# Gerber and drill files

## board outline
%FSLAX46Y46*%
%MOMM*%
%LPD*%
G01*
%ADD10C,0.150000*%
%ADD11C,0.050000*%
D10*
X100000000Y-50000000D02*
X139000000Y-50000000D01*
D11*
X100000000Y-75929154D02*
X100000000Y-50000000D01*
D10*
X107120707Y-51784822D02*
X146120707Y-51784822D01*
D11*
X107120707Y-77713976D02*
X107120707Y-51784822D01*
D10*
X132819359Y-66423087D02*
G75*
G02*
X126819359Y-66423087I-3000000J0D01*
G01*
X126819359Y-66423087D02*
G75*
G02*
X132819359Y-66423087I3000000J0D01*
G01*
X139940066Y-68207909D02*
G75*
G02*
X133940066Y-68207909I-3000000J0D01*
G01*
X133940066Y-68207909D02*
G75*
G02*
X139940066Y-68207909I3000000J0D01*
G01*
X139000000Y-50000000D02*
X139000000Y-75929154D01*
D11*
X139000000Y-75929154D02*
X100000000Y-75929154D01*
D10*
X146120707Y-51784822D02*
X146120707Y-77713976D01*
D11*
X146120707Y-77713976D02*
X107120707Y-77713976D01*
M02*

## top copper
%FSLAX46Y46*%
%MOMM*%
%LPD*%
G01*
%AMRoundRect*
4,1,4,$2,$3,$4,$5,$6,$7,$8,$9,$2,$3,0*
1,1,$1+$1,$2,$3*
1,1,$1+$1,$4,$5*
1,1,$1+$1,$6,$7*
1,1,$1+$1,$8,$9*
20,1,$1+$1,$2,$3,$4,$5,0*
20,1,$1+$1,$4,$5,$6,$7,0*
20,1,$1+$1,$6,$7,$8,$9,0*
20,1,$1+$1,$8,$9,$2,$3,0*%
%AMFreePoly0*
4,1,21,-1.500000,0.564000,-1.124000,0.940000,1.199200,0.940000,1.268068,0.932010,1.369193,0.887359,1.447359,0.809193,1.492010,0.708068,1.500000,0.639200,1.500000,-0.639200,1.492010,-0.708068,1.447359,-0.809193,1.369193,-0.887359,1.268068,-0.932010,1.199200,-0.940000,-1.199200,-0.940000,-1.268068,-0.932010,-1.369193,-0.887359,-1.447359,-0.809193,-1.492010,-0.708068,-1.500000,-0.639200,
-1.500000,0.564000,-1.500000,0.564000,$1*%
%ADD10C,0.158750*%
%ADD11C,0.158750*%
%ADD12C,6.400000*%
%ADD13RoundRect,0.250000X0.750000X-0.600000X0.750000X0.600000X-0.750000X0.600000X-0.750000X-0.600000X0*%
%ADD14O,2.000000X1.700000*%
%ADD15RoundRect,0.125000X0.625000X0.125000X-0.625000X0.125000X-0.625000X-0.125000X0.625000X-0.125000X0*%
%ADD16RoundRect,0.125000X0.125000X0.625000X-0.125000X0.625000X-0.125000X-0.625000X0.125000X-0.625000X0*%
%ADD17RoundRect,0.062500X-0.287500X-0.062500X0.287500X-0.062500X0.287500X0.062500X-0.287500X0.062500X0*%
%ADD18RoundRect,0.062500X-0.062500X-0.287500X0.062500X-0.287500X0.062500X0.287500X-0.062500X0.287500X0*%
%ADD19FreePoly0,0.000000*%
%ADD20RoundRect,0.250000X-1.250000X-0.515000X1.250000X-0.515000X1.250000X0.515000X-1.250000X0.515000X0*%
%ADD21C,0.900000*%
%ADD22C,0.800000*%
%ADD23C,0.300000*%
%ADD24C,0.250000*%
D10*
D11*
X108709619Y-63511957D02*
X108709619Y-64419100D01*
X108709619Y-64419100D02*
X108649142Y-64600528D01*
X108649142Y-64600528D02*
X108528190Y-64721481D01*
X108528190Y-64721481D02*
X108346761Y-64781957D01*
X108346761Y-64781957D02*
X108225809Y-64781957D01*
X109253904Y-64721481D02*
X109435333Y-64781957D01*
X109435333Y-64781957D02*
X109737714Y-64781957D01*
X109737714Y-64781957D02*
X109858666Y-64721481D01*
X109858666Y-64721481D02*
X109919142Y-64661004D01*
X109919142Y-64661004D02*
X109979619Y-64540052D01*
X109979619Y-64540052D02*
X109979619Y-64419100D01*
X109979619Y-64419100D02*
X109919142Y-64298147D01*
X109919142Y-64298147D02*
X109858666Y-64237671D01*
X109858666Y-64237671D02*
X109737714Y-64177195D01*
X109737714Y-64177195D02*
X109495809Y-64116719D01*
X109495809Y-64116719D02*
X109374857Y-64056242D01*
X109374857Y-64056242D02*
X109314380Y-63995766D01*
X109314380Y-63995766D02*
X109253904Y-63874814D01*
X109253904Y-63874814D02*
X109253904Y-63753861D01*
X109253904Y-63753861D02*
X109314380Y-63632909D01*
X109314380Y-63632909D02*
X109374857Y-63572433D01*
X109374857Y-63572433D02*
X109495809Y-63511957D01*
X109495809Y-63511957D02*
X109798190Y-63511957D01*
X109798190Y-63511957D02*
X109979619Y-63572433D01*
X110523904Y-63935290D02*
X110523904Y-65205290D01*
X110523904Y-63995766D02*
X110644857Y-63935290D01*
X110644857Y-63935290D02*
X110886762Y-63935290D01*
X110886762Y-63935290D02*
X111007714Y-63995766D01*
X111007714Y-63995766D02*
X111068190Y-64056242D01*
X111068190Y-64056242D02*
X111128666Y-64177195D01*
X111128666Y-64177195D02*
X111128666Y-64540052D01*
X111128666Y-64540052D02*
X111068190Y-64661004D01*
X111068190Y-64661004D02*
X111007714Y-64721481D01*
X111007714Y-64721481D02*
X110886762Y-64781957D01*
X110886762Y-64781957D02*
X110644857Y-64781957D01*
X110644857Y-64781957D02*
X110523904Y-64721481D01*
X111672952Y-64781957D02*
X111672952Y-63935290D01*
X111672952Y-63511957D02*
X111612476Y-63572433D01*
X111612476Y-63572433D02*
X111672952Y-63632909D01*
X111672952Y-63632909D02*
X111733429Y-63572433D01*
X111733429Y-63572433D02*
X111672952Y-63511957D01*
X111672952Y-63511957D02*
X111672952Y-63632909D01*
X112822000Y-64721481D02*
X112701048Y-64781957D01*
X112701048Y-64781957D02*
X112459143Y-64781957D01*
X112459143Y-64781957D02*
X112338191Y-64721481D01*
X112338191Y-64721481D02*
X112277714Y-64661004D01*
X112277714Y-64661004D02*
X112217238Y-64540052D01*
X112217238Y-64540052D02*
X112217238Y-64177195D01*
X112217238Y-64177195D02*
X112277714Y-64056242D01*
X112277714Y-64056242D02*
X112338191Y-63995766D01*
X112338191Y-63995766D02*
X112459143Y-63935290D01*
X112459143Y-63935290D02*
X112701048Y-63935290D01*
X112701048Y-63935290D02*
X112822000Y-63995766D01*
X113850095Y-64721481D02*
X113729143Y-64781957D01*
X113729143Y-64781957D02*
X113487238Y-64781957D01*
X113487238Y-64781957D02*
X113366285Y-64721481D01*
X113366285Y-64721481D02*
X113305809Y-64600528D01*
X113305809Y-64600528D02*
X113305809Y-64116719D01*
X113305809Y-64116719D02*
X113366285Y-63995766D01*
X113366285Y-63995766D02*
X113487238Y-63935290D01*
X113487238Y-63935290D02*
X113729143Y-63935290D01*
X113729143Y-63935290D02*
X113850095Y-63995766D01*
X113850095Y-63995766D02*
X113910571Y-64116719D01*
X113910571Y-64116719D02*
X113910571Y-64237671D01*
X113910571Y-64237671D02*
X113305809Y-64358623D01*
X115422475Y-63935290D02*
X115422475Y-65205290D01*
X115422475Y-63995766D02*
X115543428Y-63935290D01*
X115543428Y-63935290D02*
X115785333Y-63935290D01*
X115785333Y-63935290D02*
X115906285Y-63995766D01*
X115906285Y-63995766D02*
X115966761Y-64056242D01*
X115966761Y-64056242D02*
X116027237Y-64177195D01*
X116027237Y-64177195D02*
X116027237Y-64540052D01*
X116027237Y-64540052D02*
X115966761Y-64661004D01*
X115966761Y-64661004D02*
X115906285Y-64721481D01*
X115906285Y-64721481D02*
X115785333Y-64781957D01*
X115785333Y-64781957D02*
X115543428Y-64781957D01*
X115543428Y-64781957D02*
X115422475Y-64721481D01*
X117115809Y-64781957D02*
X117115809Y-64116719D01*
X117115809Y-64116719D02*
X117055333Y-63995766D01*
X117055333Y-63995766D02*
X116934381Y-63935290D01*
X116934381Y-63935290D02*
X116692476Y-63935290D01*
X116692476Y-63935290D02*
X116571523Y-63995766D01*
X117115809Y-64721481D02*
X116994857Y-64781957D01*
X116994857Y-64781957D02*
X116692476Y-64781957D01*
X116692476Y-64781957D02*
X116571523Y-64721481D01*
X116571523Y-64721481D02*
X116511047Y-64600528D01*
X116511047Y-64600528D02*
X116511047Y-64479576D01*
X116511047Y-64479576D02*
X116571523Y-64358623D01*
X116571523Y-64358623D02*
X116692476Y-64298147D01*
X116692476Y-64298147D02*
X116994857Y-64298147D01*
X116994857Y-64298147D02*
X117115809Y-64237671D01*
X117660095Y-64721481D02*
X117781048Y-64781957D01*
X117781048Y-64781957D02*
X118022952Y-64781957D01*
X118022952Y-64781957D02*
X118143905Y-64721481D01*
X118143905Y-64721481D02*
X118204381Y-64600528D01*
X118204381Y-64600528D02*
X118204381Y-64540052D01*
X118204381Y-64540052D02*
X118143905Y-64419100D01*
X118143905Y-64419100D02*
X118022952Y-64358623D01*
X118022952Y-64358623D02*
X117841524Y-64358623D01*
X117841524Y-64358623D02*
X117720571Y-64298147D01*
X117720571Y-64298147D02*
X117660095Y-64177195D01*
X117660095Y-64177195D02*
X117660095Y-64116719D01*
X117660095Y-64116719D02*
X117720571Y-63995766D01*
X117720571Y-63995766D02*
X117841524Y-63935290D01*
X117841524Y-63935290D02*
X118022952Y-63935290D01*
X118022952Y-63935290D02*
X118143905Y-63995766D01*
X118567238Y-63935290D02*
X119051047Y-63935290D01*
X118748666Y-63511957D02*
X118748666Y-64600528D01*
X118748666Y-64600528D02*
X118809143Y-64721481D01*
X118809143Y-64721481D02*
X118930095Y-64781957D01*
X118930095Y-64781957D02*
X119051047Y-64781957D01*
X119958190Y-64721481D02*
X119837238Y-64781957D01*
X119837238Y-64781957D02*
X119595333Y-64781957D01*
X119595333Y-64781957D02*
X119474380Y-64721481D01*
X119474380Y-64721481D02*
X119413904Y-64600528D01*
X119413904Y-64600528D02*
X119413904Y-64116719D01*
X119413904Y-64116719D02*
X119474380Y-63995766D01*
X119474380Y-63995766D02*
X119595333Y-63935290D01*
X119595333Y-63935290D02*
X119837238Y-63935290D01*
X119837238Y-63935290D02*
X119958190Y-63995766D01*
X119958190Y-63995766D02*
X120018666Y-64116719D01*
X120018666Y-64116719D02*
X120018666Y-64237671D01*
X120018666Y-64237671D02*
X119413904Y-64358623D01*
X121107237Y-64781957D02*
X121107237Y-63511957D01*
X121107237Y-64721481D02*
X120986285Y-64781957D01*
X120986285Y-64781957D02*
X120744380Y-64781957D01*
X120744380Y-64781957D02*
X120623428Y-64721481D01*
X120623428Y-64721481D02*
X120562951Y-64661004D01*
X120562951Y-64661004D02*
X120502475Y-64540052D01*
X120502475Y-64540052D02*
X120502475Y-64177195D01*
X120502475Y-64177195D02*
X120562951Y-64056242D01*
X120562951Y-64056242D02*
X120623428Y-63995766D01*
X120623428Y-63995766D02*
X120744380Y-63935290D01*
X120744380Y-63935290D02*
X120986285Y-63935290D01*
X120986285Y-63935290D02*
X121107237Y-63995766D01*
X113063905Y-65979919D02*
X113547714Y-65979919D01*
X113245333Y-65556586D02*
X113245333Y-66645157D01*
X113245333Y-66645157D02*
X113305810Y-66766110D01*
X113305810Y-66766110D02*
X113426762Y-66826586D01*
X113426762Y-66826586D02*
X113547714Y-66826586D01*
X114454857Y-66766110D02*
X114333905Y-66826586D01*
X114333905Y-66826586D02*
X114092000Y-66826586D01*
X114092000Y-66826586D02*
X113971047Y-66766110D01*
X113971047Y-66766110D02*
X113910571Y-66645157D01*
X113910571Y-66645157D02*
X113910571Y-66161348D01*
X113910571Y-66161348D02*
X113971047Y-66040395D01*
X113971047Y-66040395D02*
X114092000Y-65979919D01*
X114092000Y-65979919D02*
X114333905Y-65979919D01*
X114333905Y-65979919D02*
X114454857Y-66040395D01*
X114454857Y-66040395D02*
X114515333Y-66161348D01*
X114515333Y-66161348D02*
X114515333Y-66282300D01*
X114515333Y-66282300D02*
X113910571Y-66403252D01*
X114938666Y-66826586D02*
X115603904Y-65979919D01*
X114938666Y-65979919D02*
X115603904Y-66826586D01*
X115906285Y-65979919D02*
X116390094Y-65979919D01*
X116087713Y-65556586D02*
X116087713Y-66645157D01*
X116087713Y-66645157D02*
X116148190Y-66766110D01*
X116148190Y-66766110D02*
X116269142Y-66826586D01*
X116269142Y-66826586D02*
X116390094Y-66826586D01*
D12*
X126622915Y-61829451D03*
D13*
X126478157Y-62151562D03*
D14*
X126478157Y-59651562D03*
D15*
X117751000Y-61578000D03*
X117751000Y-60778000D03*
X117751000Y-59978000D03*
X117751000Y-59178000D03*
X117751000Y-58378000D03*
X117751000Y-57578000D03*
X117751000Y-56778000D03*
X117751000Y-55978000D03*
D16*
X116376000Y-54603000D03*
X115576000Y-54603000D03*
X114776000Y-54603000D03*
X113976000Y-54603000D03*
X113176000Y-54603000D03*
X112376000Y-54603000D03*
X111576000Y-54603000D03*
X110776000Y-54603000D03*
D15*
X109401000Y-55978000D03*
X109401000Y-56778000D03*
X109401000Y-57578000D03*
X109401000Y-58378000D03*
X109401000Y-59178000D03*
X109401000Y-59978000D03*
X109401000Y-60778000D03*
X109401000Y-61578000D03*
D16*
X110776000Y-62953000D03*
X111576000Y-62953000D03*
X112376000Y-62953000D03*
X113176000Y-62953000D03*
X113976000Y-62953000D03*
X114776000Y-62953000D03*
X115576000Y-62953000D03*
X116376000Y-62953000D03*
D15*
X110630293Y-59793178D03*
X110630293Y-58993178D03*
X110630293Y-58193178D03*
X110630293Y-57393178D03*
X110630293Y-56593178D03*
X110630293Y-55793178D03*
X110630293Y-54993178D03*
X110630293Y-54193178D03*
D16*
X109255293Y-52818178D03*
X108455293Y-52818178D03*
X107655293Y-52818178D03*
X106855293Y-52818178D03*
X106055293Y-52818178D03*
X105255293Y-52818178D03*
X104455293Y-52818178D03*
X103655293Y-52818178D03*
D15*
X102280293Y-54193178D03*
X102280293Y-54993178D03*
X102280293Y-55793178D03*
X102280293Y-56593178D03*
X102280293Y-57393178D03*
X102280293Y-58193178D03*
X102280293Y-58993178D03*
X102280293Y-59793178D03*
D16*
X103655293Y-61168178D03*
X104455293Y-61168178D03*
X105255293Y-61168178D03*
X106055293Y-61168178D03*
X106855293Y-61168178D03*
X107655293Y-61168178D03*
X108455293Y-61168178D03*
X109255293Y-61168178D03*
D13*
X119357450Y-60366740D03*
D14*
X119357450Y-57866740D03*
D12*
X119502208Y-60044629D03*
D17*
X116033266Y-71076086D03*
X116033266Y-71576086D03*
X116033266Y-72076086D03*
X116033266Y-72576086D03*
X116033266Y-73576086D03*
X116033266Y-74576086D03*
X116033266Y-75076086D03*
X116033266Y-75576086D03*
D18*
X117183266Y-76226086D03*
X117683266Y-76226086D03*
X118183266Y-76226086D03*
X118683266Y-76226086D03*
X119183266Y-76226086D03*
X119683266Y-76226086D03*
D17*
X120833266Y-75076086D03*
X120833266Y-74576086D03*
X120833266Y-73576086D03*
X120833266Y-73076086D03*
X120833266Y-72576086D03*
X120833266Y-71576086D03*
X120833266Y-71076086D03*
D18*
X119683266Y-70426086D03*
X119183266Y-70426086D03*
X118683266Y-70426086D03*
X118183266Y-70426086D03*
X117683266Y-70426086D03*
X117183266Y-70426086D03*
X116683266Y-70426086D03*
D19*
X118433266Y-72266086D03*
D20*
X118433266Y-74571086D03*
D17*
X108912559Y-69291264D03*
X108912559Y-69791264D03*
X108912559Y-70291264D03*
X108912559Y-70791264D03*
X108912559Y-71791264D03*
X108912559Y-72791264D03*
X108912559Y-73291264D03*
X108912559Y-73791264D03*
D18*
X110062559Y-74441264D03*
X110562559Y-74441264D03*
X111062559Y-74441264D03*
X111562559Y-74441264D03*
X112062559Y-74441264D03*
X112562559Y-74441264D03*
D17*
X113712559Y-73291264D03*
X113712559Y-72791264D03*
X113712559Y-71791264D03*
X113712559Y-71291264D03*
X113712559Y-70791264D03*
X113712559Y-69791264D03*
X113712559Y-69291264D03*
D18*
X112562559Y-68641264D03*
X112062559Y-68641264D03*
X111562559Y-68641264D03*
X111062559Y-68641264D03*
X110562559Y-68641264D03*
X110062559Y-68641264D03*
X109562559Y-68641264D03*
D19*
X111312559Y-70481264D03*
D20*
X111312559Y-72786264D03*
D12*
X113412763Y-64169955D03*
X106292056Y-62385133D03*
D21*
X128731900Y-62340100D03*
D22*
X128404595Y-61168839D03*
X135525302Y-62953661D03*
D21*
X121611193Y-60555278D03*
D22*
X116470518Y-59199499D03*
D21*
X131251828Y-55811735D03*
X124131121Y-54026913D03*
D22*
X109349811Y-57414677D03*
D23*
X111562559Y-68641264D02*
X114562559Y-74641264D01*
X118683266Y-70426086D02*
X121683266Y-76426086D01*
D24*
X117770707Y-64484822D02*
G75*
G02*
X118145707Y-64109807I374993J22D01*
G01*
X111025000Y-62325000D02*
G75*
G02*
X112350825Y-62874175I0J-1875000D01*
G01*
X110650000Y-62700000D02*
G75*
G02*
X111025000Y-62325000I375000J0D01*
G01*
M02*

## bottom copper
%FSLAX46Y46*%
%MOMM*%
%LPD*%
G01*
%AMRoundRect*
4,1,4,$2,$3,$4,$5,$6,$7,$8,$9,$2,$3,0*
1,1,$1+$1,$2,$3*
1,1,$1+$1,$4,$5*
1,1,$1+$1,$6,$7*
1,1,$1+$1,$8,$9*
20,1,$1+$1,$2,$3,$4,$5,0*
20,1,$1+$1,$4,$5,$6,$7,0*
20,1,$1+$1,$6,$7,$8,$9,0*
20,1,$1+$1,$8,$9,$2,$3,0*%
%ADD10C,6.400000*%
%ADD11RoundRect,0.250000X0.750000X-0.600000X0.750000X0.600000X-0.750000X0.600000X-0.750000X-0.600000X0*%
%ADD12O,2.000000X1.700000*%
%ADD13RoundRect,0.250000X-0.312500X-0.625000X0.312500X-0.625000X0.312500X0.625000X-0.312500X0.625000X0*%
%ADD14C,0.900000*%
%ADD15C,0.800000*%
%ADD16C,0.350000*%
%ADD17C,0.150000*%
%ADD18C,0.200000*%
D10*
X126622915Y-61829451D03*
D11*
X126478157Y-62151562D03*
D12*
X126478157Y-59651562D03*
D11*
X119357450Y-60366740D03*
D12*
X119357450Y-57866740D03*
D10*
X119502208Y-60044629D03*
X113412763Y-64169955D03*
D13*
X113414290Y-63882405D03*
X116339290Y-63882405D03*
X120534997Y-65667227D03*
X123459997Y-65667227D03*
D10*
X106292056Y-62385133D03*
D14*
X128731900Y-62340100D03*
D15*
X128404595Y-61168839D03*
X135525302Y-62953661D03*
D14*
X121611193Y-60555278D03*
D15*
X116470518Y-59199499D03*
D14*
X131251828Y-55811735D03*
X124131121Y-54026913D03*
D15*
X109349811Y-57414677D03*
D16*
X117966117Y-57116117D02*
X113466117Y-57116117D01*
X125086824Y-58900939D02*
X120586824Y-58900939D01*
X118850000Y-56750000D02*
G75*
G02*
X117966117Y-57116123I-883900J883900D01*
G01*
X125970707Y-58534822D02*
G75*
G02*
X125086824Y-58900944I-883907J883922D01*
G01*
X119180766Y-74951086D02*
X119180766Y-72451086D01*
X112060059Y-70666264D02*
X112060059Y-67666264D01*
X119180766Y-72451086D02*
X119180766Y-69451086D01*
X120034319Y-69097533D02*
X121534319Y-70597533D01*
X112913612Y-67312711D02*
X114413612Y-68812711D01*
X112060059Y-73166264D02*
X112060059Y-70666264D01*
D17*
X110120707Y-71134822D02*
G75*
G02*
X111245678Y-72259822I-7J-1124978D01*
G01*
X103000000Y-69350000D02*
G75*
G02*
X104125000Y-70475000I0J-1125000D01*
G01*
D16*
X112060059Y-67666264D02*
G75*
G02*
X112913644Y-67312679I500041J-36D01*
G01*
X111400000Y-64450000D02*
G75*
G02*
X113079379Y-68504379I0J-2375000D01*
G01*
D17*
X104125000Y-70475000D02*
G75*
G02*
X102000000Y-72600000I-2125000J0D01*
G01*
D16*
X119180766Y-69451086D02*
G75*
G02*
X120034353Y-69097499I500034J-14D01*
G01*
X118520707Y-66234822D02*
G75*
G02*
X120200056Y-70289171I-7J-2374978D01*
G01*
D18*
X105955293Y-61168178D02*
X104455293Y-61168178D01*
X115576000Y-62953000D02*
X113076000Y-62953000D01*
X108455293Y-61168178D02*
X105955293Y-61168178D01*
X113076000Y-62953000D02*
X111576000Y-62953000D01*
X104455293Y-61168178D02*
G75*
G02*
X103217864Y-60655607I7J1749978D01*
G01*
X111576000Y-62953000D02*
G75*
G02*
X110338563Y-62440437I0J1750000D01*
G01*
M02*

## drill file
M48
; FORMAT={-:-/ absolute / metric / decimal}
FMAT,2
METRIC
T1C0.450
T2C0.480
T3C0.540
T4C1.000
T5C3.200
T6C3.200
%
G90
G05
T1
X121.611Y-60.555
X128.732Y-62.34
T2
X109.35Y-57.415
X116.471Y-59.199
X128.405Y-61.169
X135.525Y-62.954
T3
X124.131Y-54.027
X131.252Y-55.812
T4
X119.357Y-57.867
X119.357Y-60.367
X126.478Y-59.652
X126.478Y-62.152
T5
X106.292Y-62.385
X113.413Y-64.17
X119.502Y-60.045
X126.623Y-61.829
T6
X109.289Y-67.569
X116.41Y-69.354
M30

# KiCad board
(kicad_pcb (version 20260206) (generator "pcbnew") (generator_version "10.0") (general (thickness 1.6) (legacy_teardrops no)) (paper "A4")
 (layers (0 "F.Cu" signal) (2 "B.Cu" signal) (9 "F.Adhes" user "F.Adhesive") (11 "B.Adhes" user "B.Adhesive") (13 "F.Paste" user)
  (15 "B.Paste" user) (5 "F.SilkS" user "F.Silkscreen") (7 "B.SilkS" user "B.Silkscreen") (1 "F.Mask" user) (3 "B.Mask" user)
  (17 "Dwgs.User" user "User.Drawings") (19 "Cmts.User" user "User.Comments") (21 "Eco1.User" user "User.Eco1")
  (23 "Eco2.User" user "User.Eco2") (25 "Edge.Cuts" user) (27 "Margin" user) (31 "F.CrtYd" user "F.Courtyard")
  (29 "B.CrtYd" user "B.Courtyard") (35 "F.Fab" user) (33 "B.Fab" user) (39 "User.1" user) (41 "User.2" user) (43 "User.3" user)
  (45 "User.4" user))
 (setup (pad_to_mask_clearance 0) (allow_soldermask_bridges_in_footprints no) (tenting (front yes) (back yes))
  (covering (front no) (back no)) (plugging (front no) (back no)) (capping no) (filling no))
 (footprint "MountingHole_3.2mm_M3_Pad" (layer "F.Cu") (at 126.622915 61.829451)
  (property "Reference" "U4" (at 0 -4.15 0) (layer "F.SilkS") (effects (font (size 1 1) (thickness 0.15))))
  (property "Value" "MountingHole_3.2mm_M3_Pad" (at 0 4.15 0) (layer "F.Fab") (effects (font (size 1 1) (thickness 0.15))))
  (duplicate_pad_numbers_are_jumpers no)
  (pad "1" thru_hole circle (at 0 0) (size 6.4 6.4) (drill 3.2) (layers "*.Cu" "*.Mask") (remove_unused_layers no) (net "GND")
   (zone_connect 2)))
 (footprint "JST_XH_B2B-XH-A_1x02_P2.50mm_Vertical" (layer "F.Cu") (at 126.478157 62.151562 90)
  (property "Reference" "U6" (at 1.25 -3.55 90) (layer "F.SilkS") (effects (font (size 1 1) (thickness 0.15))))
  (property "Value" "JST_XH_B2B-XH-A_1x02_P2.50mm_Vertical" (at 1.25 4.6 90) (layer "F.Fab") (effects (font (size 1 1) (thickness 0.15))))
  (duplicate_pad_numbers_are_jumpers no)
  (pad "1" thru_hole roundrect (at 0 0 90) (size 1.7 2) (drill 1) (layers "*.Cu" "*.Mask") (remove_unused_layers no)
   (roundrect_rratio 0.147059) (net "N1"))
  (pad "2" thru_hole oval (at 2.5 0 90) (size 1.7 2) (drill 1) (layers "*.Cu" "*.Mask") (remove_unused_layers no)))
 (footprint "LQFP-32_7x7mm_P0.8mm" (layer "F.Cu") (at 113.576 58.778 180)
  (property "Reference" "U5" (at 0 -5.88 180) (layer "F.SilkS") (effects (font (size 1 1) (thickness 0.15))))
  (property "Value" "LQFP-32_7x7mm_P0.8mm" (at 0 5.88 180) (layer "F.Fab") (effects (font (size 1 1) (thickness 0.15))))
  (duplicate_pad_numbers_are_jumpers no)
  (pad "1" smd roundrect (at -4.175 -2.8 180) (size 1.5 0.5) (layers "F.Cu" "F.Mask" "F.Paste") (roundrect_rratio 0.25) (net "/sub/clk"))
  (pad "2" smd roundrect (at -4.175 -2 180) (size 1.5 0.5) (layers "F.Cu" "F.Mask" "F.Paste") (roundrect_rratio 0.25) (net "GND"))
  (pad "3" smd roundrect (at -4.175 -1.2 180) (size 1.5 0.5) (layers "F.Cu" "F.Mask" "F.Paste") (roundrect_rratio 0.25) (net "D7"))
  (pad "4" smd roundrect (at -4.175 -0.4 180) (size 1.5 0.5) (layers "F.Cu" "F.Mask" "F.Paste") (roundrect_rratio 0.25) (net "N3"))
  (pad "5" smd roundrect (at -4.175 0.4 180) (size 1.5 0.5) (layers "F.Cu" "F.Mask" "F.Paste") (roundrect_rratio 0.25))
  (pad "6" smd roundrect (at -4.175 1.2 180) (size 1.5 0.5) (layers "F.Cu" "F.Mask" "F.Paste") (roundrect_rratio 0.25) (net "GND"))
  (pad "7" smd roundrect (at -4.175 2 180) (size 1.5 0.5) (layers "F.Cu" "F.Mask" "F.Paste") (roundrect_rratio 0.25))
  (pad "8" smd roundrect (at -4.175 2.8 180) (size 1.5 0.5) (layers "F.Cu" "F.Mask" "F.Paste") (roundrect_rratio 0.25) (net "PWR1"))
  (pad "9" smd roundrect (at -2.8 4.175 180) (size 0.5 1.5) (layers "F.Cu" "F.Mask" "F.Paste") (roundrect_rratio 0.25) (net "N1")
   (clearance 0.35))
  (pad "10" smd roundrect (at -2 4.175 180) (size 0.5 1.5) (layers "F.Cu" "F.Mask" "F.Paste") (roundrect_rratio 0.25) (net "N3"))
  (pad "11" smd roundrect (at -1.2 4.175 180) (size 0.5 1.5) (layers "F.Cu" "F.Mask" "F.Paste") (roundrect_rratio 0.25) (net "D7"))
  (pad "12" smd roundrect (at -0.4 4.175 180) (size 0.5 1.5) (layers "F.Cu" "F.Mask" "F.Paste") (roundrect_rratio 0.25) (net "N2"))
  (pad "13" smd roundrect (at 0.4 4.175 180) (size 0.5 1.5) (layers "F.Cu" "F.Mask" "F.Paste") (roundrect_rratio 0.25) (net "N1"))
  (pad "14" smd roundrect (at 1.2 4.175 180) (size 0.5 1.5) (layers "F.Cu" "F.Mask" "F.Paste") (roundrect_rratio 0.25) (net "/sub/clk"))
  (pad "15" smd roundrect (at 2 4.175 180) (size 0.5 1.5) (layers "F.Cu" "F.Mask" "F.Paste") (roundrect_rratio 0.25))
  (pad "16" smd roundrect (at 2.8 4.175 180) (size 0.5 1.5) (layers "F.Cu" "F.Mask" "F.Paste") (roundrect_rratio 0.25))
  (pad "17" smd roundrect (at 4.175 2.8 180) (size 1.5 0.5) (layers "F.Cu" "F.Mask" "F.Paste") (roundrect_rratio 0.25) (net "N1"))
  (pad "18" smd roundrect (at 4.175 2 180) (size 1.5 0.5) (layers "F.Cu" "F.Mask" "F.Paste") (roundrect_rratio 0.25) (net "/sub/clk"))
  (pad "19" smd roundrect (at 4.175 1.2 180) (size 1.5 0.5) (layers "F.Cu" "F.Mask" "F.Paste") (roundrect_rratio 0.25) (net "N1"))
  (pad "20" smd roundrect (at 4.175 0.4 180) (size 1.5 0.5) (layers "F.Cu" "F.Mask" "F.Paste") (roundrect_rratio 0.25) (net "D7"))
  (pad "21" smd roundrect (at 4.175 -0.4 180) (size 1.5 0.5) (layers "F.Cu" "F.Mask" "F.Paste") (roundrect_rratio 0.25) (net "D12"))
  (pad "22" smd roundrect (at 4.175 -1.2 180) (size 1.5 0.5) (layers "F.Cu" "F.Mask" "F.Paste") (roundrect_rratio 0.25))
  (pad "23" smd roundrect (at 4.175 -2 180) (size 1.5 0.5) (layers "F.Cu" "F.Mask" "F.Paste") (roundrect_rratio 0.25))
  (pad "24" smd roundrect (at 4.175 -2.8 180) (size 1.5 0.5) (layers "F.Cu" "F.Mask" "F.Paste") (roundrect_rratio 0.25))
  (pad "25" smd roundrect (at 2.8 -4.175 180) (size 0.5 1.5) (layers "F.Cu" "F.Mask" "F.Paste") (roundrect_rratio 0.25) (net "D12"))
  (pad "26" smd roundrect (at 2 -4.175 180) (size 0.5 1.5) (layers "F.Cu" "F.Mask" "F.Paste") (roundrect_rratio 0.25) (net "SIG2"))
  (pad "27" smd roundrect (at 1.2 -4.175 180) (size 0.5 1.5) (layers "F.Cu" "F.Mask" "F.Paste") (roundrect_rratio 0.25) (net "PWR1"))
  (pad "28" smd roundrect (at 0.4 -4.175 180) (size 0.5 1.5) (layers "F.Cu" "F.Mask" "F.Paste") (roundrect_rratio 0.25) (clearance 0.35))
  (pad "29" smd roundrect (at -0.4 -4.175 180) (size 0.5 1.5) (layers "F.Cu" "F.Mask" "F.Paste") (roundrect_rratio 0.25) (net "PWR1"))
  (pad "30" smd roundrect (at -1.2 -4.175 180) (size 0.5 1.5) (layers "F.Cu" "F.Mask" "F.Paste") (roundrect_rratio 0.25) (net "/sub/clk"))
  (pad "31" smd roundrect (at -2 -4.175 180) (size 0.5 1.5) (layers "F.Cu" "F.Mask" "F.Paste") (roundrect_rratio 0.25) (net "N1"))
  (pad "32" smd roundrect (at -2.8 -4.175 180) (size 0.5 1.5) (layers "F.Cu" "F.Mask" "F.Paste") (roundrect_rratio 0.25) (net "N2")))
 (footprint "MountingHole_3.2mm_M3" (layer "F.Cu") (at 109.289246 67.568769)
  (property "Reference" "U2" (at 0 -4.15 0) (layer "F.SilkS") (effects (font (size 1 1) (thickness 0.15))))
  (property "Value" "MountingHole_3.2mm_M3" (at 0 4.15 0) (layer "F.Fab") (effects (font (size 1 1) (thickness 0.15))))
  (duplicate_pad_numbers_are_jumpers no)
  (pad "" np_thru_hole circle (at 0 0) (size 3.2 3.2) (drill 3.2) (layers "*.Cu" "*.Mask")))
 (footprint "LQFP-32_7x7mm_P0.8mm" (layer "F.Cu") (at 106.455293 56.993178 180)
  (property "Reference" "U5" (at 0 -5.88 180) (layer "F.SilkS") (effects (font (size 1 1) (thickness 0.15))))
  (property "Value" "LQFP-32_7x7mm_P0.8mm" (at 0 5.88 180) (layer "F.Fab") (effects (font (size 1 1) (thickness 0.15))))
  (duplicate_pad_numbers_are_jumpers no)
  (pad "1" smd roundrect (at -4.175 -2.8 180) (size 1.5 0.5) (layers "F.Cu" "F.Mask" "F.Paste") (roundrect_rratio 0.25) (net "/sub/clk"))
  (pad "2" smd roundrect (at -4.175 -2 180) (size 1.5 0.5) (layers "F.Cu" "F.Mask" "F.Paste") (roundrect_rratio 0.25) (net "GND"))
  (pad "3" smd roundrect (at -4.175 -1.2 180) (size 1.5 0.5) (layers "F.Cu" "F.Mask" "F.Paste") (roundrect_rratio 0.25) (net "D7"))
  (pad "4" smd roundrect (at -4.175 -0.4 180) (size 1.5 0.5) (layers "F.Cu" "F.Mask" "F.Paste") (roundrect_rratio 0.25) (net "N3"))
  (pad "5" smd roundrect (at -4.175 0.4 180) (size 1.5 0.5) (layers "F.Cu" "F.Mask" "F.Paste") (roundrect_rratio 0.25))
  (pad "6" smd roundrect (at -4.175 1.2 180) (size 1.5 0.5) (layers "F.Cu" "F.Mask" "F.Paste") (roundrect_rratio 0.25) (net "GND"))
  (pad "7" smd roundrect (at -4.175 2 180) (size 1.5 0.5) (layers "F.Cu" "F.Mask" "F.Paste") (roundrect_rratio 0.25))
  (pad "8" smd roundrect (at -4.175 2.8 180) (size 1.5 0.5) (layers "F.Cu" "F.Mask" "F.Paste") (roundrect_rratio 0.25) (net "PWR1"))
  (pad "9" smd roundrect (at -2.8 4.175 180) (size 0.5 1.5) (layers "F.Cu" "F.Mask" "F.Paste") (roundrect_rratio 0.25) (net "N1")
   (clearance 0.35))
  (pad "10" smd roundrect (at -2 4.175 180) (size 0.5 1.5) (layers "F.Cu" "F.Mask" "F.Paste") (roundrect_rratio 0.25) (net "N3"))
  (pad "11" smd roundrect (at -1.2 4.175 180) (size 0.5 1.5) (layers "F.Cu" "F.Mask" "F.Paste") (roundrect_rratio 0.25) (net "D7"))
  (pad "12" smd roundrect (at -0.4 4.175 180) (size 0.5 1.5) (layers "F.Cu" "F.Mask" "F.Paste") (roundrect_rratio 0.25) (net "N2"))
  (pad "13" smd roundrect (at 0.4 4.175 180) (size 0.5 1.5) (layers "F.Cu" "F.Mask" "F.Paste") (roundrect_rratio 0.25) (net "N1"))
  (pad "14" smd roundrect (at 1.2 4.175 180) (size 0.5 1.5) (layers "F.Cu" "F.Mask" "F.Paste") (roundrect_rratio 0.25) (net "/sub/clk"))
  (pad "15" smd roundrect (at 2 4.175 180) (size 0.5 1.5) (layers "F.Cu" "F.Mask" "F.Paste") (roundrect_rratio 0.25))
  (pad "16" smd roundrect (at 2.8 4.175 180) (size 0.5 1.5) (layers "F.Cu" "F.Mask" "F.Paste") (roundrect_rratio 0.25))
  (pad "17" smd roundrect (at 4.175 2.8 180) (size 1.5 0.5) (layers "F.Cu" "F.Mask" "F.Paste") (roundrect_rratio 0.25) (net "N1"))
  (pad "18" smd roundrect (at 4.175 2 180) (size 1.5 0.5) (layers "F.Cu" "F.Mask" "F.Paste") (roundrect_rratio 0.25) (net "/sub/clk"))
  (pad "19" smd roundrect (at 4.175 1.2 180) (size 1.5 0.5) (layers "F.Cu" "F.Mask" "F.Paste") (roundrect_rratio 0.25) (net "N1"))
  (pad "20" smd roundrect (at 4.175 0.4 180) (size 1.5 0.5) (layers "F.Cu" "F.Mask" "F.Paste") (roundrect_rratio 0.25) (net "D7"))
  (pad "21" smd roundrect (at 4.175 -0.4 180) (size 1.5 0.5) (layers "F.Cu" "F.Mask" "F.Paste") (roundrect_rratio 0.25) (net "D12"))
  (pad "22" smd roundrect (at 4.175 -1.2 180) (size 1.5 0.5) (layers "F.Cu" "F.Mask" "F.Paste") (roundrect_rratio 0.25))
  (pad "23" smd roundrect (at 4.175 -2 180) (size 1.5 0.5) (layers "F.Cu" "F.Mask" "F.Paste") (roundrect_rratio 0.25))
  (pad "24" smd roundrect (at 4.175 -2.8 180) (size 1.5 0.5) (layers "F.Cu" "F.Mask" "F.Paste") (roundrect_rratio 0.25))
  (pad "25" smd roundrect (at 2.8 -4.175 180) (size 0.5 1.5) (layers "F.Cu" "F.Mask" "F.Paste") (roundrect_rratio 0.25) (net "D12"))
  (pad "26" smd roundrect (at 2 -4.175 180) (size 0.5 1.5) (layers "F.Cu" "F.Mask" "F.Paste") (roundrect_rratio 0.25) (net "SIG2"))
  (pad "27" smd roundrect (at 1.2 -4.175 180) (size 0.5 1.5) (layers "F.Cu" "F.Mask" "F.Paste") (roundrect_rratio 0.25) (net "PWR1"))
  (pad "28" smd roundrect (at 0.4 -4.175 180) (size 0.5 1.5) (layers "F.Cu" "F.Mask" "F.Paste") (roundrect_rratio 0.25) (clearance 0.35))
  (pad "29" smd roundrect (at -0.4 -4.175 180) (size 0.5 1.5) (layers "F.Cu" "F.Mask" "F.Paste") (roundrect_rratio 0.25) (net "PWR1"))
  (pad "30" smd roundrect (at -1.2 -4.175 180) (size 0.5 1.5) (layers "F.Cu" "F.Mask" "F.Paste") (roundrect_rratio 0.25) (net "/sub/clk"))
  (pad "31" smd roundrect (at -2 -4.175 180) (size 0.5 1.5) (layers "F.Cu" "F.Mask" "F.Paste") (roundrect_rratio 0.25) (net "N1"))
  (pad "32" smd roundrect (at -2.8 -4.175 180) (size 0.5 1.5) (layers "F.Cu" "F.Mask" "F.Paste") (roundrect_rratio 0.25) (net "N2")))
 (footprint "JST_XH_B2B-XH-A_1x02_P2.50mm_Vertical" (layer "F.Cu") (at 119.35745 60.36674 90)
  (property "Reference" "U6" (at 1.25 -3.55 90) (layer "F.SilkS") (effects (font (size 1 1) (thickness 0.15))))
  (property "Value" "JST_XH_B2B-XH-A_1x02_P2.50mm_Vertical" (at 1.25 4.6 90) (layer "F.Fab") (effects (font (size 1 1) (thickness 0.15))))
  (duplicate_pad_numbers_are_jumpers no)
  (pad "1" thru_hole roundrect (at 0 0 90) (size 1.7 2) (drill 1) (layers "*.Cu" "*.Mask") (remove_unused_layers no)
   (roundrect_rratio 0.147059) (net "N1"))
  (pad "2" thru_hole oval (at 2.5 0 90) (size 1.7 2) (drill 1) (layers "*.Cu" "*.Mask") (remove_unused_layers no)))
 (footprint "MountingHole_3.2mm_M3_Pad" (layer "F.Cu") (at 119.502208 60.044629)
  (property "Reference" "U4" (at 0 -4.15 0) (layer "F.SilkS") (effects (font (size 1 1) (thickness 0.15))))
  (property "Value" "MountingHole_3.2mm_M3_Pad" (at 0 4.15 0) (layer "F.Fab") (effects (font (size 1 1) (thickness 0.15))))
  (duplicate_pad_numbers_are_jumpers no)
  (pad "1" thru_hole circle (at 0 0) (size 6.4 6.4) (drill 3.2) (layers "*.Cu" "*.Mask") (remove_unused_layers no) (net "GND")
   (zone_connect 2)))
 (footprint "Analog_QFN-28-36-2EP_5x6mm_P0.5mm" (layer "F.Cu") (at 118.433266 73.326086)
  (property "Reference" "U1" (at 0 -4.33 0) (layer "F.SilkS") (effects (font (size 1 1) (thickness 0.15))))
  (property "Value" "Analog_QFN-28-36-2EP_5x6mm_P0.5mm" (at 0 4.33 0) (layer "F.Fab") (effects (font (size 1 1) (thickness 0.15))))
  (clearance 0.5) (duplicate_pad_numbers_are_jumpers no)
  (pad "" smd roundrect (at -0.75 -1.53) (size 1.21 0.76) (layers "F.Paste") (roundrect_rratio 0.25) (chamfer_ratio 0.4) (chamfer top_left)
   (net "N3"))
  (pad "" smd roundrect (at -0.75 -0.59) (size 1.21 0.76) (layers "F.Paste") (roundrect_rratio 0.25) (clearance 0.1))
  (pad "" smd roundrect (at -0.7475 0.875) (size 1.205 0.55) (layers "F.Paste") (roundrect_rratio 0.25) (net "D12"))
  (pad "" smd roundrect (at -0.7475 1.625) (size 1.205 0.55) (layers "F.Paste") (roundrect_rratio 0.25) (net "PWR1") (clearance 0.35))
  (pad "" smd roundrect (at 0.7475 0.875) (size 1.205 0.55) (layers "F.Paste") (roundrect_rratio 0.25) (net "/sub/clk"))
  (pad "" smd roundrect (at 0.7475 1.625) (size 1.205 0.55) (layers "F.Paste") (roundrect_rratio 0.25) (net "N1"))
  (pad "" smd roundrect (at 0.75 -1.53) (size 1.21 0.76) (layers "F.Paste") (roundrect_rratio 0.25) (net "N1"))
  (pad "" smd roundrect (at 0.75 -0.59) (size 1.21 0.76) (layers "F.Paste") (roundrect_rratio 0.25) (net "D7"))
  (pad "1" smd roundrect (at -2.4 -2.25) (size 0.7 0.25) (layers "F.Cu" "F.Mask" "F.Paste") (roundrect_rratio 0.25) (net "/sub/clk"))
  (pad "2" smd roundrect (at -2.4 -1.75) (size 0.7 0.25) (layers "F.Cu" "F.Mask" "F.Paste") (roundrect_rratio 0.25) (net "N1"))
  (pad "3" smd roundrect (at -2.4 -1.25) (size 0.7 0.25) (layers "F.Cu" "F.Mask" "F.Paste") (roundrect_rratio 0.25))
  (pad "4" smd roundrect (at -2.4 -0.75) (size 0.7 0.25) (layers "F.Cu" "F.Mask" "F.Paste") (roundrect_rratio 0.25))
  (pad "6" smd roundrect (at -2.4 0.25) (size 0.7 0.25) (layers "F.Cu" "F.Mask" "F.Paste") (roundrect_rratio 0.25) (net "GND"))
  (pad "8" smd roundrect (at -2.4 1.25) (size 0.7 0.25) (layers "F.Cu" "F.Mask" "F.Paste") (roundrect_rratio 0.25))
  (pad "9" smd roundrect (at -2.4 1.75) (size 0.7 0.25) (layers "F.Cu" "F.Mask" "F.Paste") (roundrect_rratio 0.25) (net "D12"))
  (pad "10" smd roundrect (at -2.4 2.25) (size 0.7 0.25) (layers "F.Cu" "F.Mask" "F.Paste") (roundrect_rratio 0.25) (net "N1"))
  (pad "12" smd roundrect (at -1.25 2.9) (size 0.25 0.7) (layers "F.Cu" "F.Mask" "F.Paste") (roundrect_rratio 0.25))
  (pad "13" smd roundrect (at -0.75 2.9) (size 0.25 0.7) (layers "F.Cu" "F.Mask" "F.Paste") (roundrect_rratio 0.25) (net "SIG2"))
  (pad "14" smd roundrect (at -0.25 2.9) (size 0.25 0.7) (layers "F.Cu" "F.Mask" "F.Paste") (roundrect_rratio 0.25) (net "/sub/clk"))
  (pad "15" smd roundrect (at 0.25 2.9) (size 0.25 0.7) (layers "F.Cu" "F.Mask" "F.Paste") (roundrect_rratio 0.25))
  (pad "16" smd roundrect (at 0.75 2.9) (size 0.25 0.7) (layers "F.Cu" "F.Mask" "F.Paste") (roundrect_rratio 0.25) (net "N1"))
  (pad "17" smd roundrect (at 1.25 2.9) (size 0.25 0.7) (layers "F.Cu" "F.Mask" "F.Paste") (roundrect_rratio 0.25) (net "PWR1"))
  (pad "20" smd roundrect (at 2.4 1.75) (size 0.7 0.25) (layers "F.Cu" "F.Mask" "F.Paste") (roundrect_rratio 0.25) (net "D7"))
  (pad "21" smd roundrect (at 2.4 1.25) (size 0.7 0.25) (layers "F.Cu" "F.Mask" "F.Paste") (roundrect_rratio 0.25) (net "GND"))
  (pad "23" smd roundrect (at 2.4 0.25) (size 0.7 0.25) (layers "F.Cu" "F.Mask" "F.Paste") (roundrect_rratio 0.25))
  (pad "24" smd roundrect (at 2.4 -0.25) (size 0.7 0.25) (layers "F.Cu" "F.Mask" "F.Paste") (roundrect_rratio 0.25) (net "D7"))
  (pad "25" smd roundrect (at 2.4 -0.75) (size 0.7 0.25) (layers "F.Cu" "F.Mask" "F.Paste") (roundrect_rratio 0.25) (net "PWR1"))
  (pad "27" smd roundrect (at 2.4 -1.75) (size 0.7 0.25) (layers "F.Cu" "F.Mask" "F.Paste") (roundrect_rratio 0.25) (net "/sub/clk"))
  (pad "28" smd roundrect (at 2.4 -2.25) (size 0.7 0.25) (layers "F.Cu" "F.Mask" "F.Paste") (roundrect_rratio 0.25) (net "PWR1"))
  (pad "30" smd roundrect (at 1.25 -2.9) (size 0.25 0.7) (layers "F.Cu" "F.Mask" "F.Paste") (roundrect_rratio 0.25))
  (pad "31" smd roundrect (at 0.75 -2.9) (size 0.25 0.7) (layers "F.Cu" "F.Mask" "F.Paste") (roundrect_rratio 0.25))
  (pad "32" smd roundrect (at 0.25 -2.9) (size 0.25 0.7) (layers "F.Cu" "F.Mask" "F.Paste") (roundrect_rratio 0.25))
  (pad "33" smd roundrect (at -0.25 -2.9) (size 0.25 0.7) (layers "F.Cu" "F.Mask" "F.Paste") (roundrect_rratio 0.25) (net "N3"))
  (pad "34" smd roundrect (at -0.75 -2.9) (size 0.25 0.7) (layers "F.Cu" "F.Mask" "F.Paste") (roundrect_rratio 0.25))
  (pad "35" smd roundrect (at -1.25 -2.9) (size 0.25 0.7) (layers "F.Cu" "F.Mask" "F.Paste") (roundrect_rratio 0.25))
  (pad "36" smd roundrect (at -1.75 -2.9) (size 0.25 0.7) (layers "F.Cu" "F.Mask" "F.Paste") (roundrect_rratio 0.25) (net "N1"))
  (pad "37" smd roundrect (at 0 -1.06) (size 3 1.88) (layers "F.Cu" "F.Mask") (roundrect_rratio 0.16) (chamfer_ratio 0.2) (chamfer top_left)
   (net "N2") (zone_connect 2))
  (pad "38" smd roundrect (at 0 1.245) (size 3 1.53) (layers "F.Cu" "F.Mask") (roundrect_rratio 0.1633986928) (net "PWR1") (zone_connect 2)))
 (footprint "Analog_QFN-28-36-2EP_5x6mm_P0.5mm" (layer "F.Cu") (at 111.312559 71.541264)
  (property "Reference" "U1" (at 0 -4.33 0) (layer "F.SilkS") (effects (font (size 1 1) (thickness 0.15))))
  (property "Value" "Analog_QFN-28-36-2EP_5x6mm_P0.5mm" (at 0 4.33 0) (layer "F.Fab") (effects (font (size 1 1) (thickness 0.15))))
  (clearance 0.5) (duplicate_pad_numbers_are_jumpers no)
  (pad "" smd roundrect (at -0.75 -1.53) (size 1.21 0.76) (layers "F.Paste") (roundrect_rratio 0.25) (chamfer_ratio 0.4) (chamfer top_left)
   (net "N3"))
  (pad "" smd roundrect (at -0.75 -0.59) (size 1.21 0.76) (layers "F.Paste") (roundrect_rratio 0.25) (clearance 0.1))
  (pad "" smd roundrect (at -0.7475 0.875) (size 1.205 0.55) (layers "F.Paste") (roundrect_rratio 0.25) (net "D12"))
  (pad "" smd roundrect (at -0.7475 1.625) (size 1.205 0.55) (layers "F.Paste") (roundrect_rratio 0.25) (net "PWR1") (clearance 0.35))
  (pad "" smd roundrect (at 0.7475 0.875) (size 1.205 0.55) (layers "F.Paste") (roundrect_rratio 0.25) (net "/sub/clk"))
  (pad "" smd roundrect (at 0.7475 1.625) (size 1.205 0.55) (layers "F.Paste") (roundrect_rratio 0.25) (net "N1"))
  (pad "" smd roundrect (at 0.75 -1.53) (size 1.21 0.76) (layers "F.Paste") (roundrect_rratio 0.25) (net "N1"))
  (pad "" smd roundrect (at 0.75 -0.59) (size 1.21 0.76) (layers "F.Paste") (roundrect_rratio 0.25) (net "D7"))
  (pad "1" smd roundrect (at -2.4 -2.25) (size 0.7 0.25) (layers "F.Cu" "F.Mask" "F.Paste") (roundrect_rratio 0.25) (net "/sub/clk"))
  (pad "2" smd roundrect (at -2.4 -1.75) (size 0.7 0.25) (layers "F.Cu" "F.Mask" "F.Paste") (roundrect_rratio 0.25) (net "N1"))
  (pad "3" smd roundrect (at -2.4 -1.25) (size 0.7 0.25) (layers "F.Cu" "F.Mask" "F.Paste") (roundrect_rratio 0.25))
  (pad "4" smd roundrect (at -2.4 -0.75) (size 0.7 0.25) (layers "F.Cu" "F.Mask" "F.Paste") (roundrect_rratio 0.25))
  (pad "6" smd roundrect (at -2.4 0.25) (size 0.7 0.25) (layers "F.Cu" "F.Mask" "F.Paste") (roundrect_rratio 0.25) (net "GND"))
  (pad "8" smd roundrect (at -2.4 1.25) (size 0.7 0.25) (layers "F.Cu" "F.Mask" "F.Paste") (roundrect_rratio 0.25))
  (pad "9" smd roundrect (at -2.4 1.75) (size 0.7 0.25) (layers "F.Cu" "F.Mask" "F.Paste") (roundrect_rratio 0.25) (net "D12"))
  (pad "10" smd roundrect (at -2.4 2.25) (size 0.7 0.25) (layers "F.Cu" "F.Mask" "F.Paste") (roundrect_rratio 0.25) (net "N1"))
  (pad "12" smd roundrect (at -1.25 2.9) (size 0.25 0.7) (layers "F.Cu" "F.Mask" "F.Paste") (roundrect_rratio 0.25))
  (pad "13" smd roundrect (at -0.75 2.9) (size 0.25 0.7) (layers "F.Cu" "F.Mask" "F.Paste") (roundrect_rratio 0.25) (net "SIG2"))
  (pad "14" smd roundrect (at -0.25 2.9) (size 0.25 0.7) (layers "F.Cu" "F.Mask" "F.Paste") (roundrect_rratio 0.25) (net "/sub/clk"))
  (pad "15" smd roundrect (at 0.25 2.9) (size 0.25 0.7) (layers "F.Cu" "F.Mask" "F.Paste") (roundrect_rratio 0.25))
  (pad "16" smd roundrect (at 0.75 2.9) (size 0.25 0.7) (layers "F.Cu" "F.Mask" "F.Paste") (roundrect_rratio 0.25) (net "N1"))
  (pad "17" smd roundrect (at 1.25 2.9) (size 0.25 0.7) (layers "F.Cu" "F.Mask" "F.Paste") (roundrect_rratio 0.25) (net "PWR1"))
  (pad "20" smd roundrect (at 2.4 1.75) (size 0.7 0.25) (layers "F.Cu" "F.Mask" "F.Paste") (roundrect_rratio 0.25) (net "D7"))
  (pad "21" smd roundrect (at 2.4 1.25) (size 0.7 0.25) (layers "F.Cu" "F.Mask" "F.Paste") (roundrect_rratio 0.25) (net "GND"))
  (pad "23" smd roundrect (at 2.4 0.25) (size 0.7 0.25) (layers "F.Cu" "F.Mask" "F.Paste") (roundrect_rratio 0.25))
  (pad "24" smd roundrect (at 2.4 -0.25) (size 0.7 0.25) (layers "F.Cu" "F.Mask" "F.Paste") (roundrect_rratio 0.25) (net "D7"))
  (pad "25" smd roundrect (at 2.4 -0.75) (size 0.7 0.25) (layers "F.Cu" "F.Mask" "F.Paste") (roundrect_rratio 0.25) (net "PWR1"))
  (pad "27" smd roundrect (at 2.4 -1.75) (size 0.7 0.25) (layers "F.Cu" "F.Mask" "F.Paste") (roundrect_rratio 0.25) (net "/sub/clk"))
  (pad "28" smd roundrect (at 2.4 -2.25) (size 0.7 0.25) (layers "F.Cu" "F.Mask" "F.Paste") (roundrect_rratio 0.25) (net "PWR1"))
  (pad "30" smd roundrect (at 1.25 -2.9) (size 0.25 0.7) (layers "F.Cu" "F.Mask" "F.Paste") (roundrect_rratio 0.25))
  (pad "31" smd roundrect (at 0.75 -2.9) (size 0.25 0.7) (layers "F.Cu" "F.Mask" "F.Paste") (roundrect_rratio 0.25))
  (pad "32" smd roundrect (at 0.25 -2.9) (size 0.25 0.7) (layers "F.Cu" "F.Mask" "F.Paste") (roundrect_rratio 0.25))
  (pad "33" smd roundrect (at -0.25 -2.9) (size 0.25 0.7) (layers "F.Cu" "F.Mask" "F.Paste") (roundrect_rratio 0.25) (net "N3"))
  (pad "34" smd roundrect (at -0.75 -2.9) (size 0.25 0.7) (layers "F.Cu" "F.Mask" "F.Paste") (roundrect_rratio 0.25))
  (pad "35" smd roundrect (at -1.25 -2.9) (size 0.25 0.7) (layers "F.Cu" "F.Mask" "F.Paste") (roundrect_rratio 0.25))
  (pad "36" smd roundrect (at -1.75 -2.9) (size 0.25 0.7) (layers "F.Cu" "F.Mask" "F.Paste") (roundrect_rratio 0.25) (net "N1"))
  (pad "37" smd roundrect (at 0 -1.06) (size 3 1.88) (layers "F.Cu" "F.Mask") (roundrect_rratio 0.16) (chamfer_ratio 0.2) (chamfer top_left)
   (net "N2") (zone_connect 2))
  (pad "38" smd roundrect (at 0 1.245) (size 3 1.53) (layers "F.Cu" "F.Mask") (roundrect_rratio 0.1633986928) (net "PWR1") (zone_connect 2)))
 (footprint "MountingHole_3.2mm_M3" (layer "F.Cu") (at 116.409953 69.353591)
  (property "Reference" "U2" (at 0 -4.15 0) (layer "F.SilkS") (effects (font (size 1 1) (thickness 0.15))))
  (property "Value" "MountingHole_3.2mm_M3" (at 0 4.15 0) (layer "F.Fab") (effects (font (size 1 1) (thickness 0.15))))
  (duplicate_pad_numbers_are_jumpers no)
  (pad "" np_thru_hole circle (at 0 0) (size 3.2 3.2) (drill 3.2) (layers "*.Cu" "*.Mask")))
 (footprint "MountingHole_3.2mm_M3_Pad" (layer "B.Cu") (at 113.412763 64.169955 90)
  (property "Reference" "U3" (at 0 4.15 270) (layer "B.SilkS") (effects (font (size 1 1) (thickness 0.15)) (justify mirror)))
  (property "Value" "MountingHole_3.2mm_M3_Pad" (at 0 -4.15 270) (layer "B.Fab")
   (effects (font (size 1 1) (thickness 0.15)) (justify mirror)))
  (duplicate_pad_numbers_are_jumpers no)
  (pad "1" thru_hole circle (at 0 0 90) (size 6.4 6.4) (drill 3.2) (layers "*.Cu" "*.Mask") (remove_unused_layers no) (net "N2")
   (clearance 0.1) (zone_connect 2)))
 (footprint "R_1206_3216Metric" (layer "B.Cu") (at 114.87679 63.882405)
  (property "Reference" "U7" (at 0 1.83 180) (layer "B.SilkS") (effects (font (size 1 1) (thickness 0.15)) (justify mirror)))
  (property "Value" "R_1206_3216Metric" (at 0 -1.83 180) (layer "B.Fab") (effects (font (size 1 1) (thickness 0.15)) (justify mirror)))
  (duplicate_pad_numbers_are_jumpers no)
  (pad "1" smd roundrect (at -1.4625 0) (size 1.125 1.75) (layers "B.Cu" "B.Mask" "B.Paste") (roundrect_rratio 0.222222) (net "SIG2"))
  (pad "2" smd roundrect (at 1.4625 0) (size 1.125 1.75) (layers "B.Cu" "B.Mask" "B.Paste") (roundrect_rratio 0.222222) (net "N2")))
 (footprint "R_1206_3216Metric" (layer "B.Cu") (at 121.997497 65.667227)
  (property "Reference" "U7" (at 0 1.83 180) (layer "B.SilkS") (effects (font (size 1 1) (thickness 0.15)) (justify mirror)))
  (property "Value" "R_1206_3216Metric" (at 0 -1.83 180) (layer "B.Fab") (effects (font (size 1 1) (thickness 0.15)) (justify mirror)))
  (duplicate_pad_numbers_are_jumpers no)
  (pad "1" smd roundrect (at -1.4625 0) (size 1.125 1.75) (layers "B.Cu" "B.Mask" "B.Paste") (roundrect_rratio 0.222222) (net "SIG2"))
  (pad "2" smd roundrect (at 1.4625 0) (size 1.125 1.75) (layers "B.Cu" "B.Mask" "B.Paste") (roundrect_rratio 0.222222) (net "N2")))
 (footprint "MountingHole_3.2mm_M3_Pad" (layer "B.Cu") (at 106.292056 62.385133 90)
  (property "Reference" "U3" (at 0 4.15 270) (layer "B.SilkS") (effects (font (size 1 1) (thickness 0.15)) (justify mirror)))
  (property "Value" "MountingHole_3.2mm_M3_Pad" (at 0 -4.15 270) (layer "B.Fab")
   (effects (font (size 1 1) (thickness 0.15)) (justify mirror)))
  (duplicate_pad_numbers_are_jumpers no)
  (pad "1" thru_hole circle (at 0 0 90) (size 6.4 6.4) (drill 3.2) (layers "*.Cu" "*.Mask") (remove_unused_layers no) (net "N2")
   (clearance 0.1) (zone_connect 2)))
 (gr_line (start 100 50) (end 139 50) (stroke (width 0.15) (type default)) (layer "Edge.Cuts"))
 (gr_line (start 100 75.929154) (end 100 50) (stroke (width 0.05) (type default)) (layer "Edge.Cuts"))
 (gr_line (start 107.120707 51.784822) (end 146.120707 51.784822) (stroke (width 0.15) (type default)) (layer "Edge.Cuts"))
 (gr_line (start 107.120707 77.713976) (end 107.120707 51.784822) (stroke (width 0.05) (type default)) (layer "Edge.Cuts"))
 (gr_circle (center 129.819359 66.423087) (end 132.819359 66.423087) (stroke (width 0.15) (type default)) (fill no) (layer "Edge.Cuts"))
 (gr_circle (center 136.940066 68.207909) (end 139.940066 68.207909) (stroke (width 0.15) (type default)) (fill no) (layer "Edge.Cuts"))
 (gr_line (start 139 50) (end 139 75.929154) (stroke (width 0.15) (type default)) (layer "Edge.Cuts"))
 (gr_line (start 139 75.929154) (end 100 75.929154) (stroke (width 0.05) (type default)) (layer "Edge.Cuts"))
 (gr_line (start 146.120707 51.784822) (end 146.120707 77.713976) (stroke (width 0.15) (type default)) (layer "Edge.Cuts"))
 (gr_line (start 146.120707 77.713976) (end 107.120707 77.713976) (stroke (width 0.05) (type default)) (layer "Edge.Cuts"))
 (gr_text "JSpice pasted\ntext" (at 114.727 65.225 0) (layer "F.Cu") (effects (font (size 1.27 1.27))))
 (segment (start 111.562559 68.641264) (end 114.562559 74.641264) (width 0.3) (layer "F.Cu") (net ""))
 (segment (start 118.683266 70.426086) (end 121.683266 76.426086) (width 0.3) (layer "F.Cu") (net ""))
 (arc (start 117.770707 64.484822) (mid 117.880542 64.219657) (end 118.145707 64.109822) (width 0.25) (layer "F.Cu") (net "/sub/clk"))
 (arc (start 111.025 62.325) (mid 111.742531 62.467726) (end 112.350825 62.874175) (width 0.25) (locked yes) (layer "F.Cu") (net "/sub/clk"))
 (arc (start 110.65 62.7) (mid 110.759835 62.434835) (end 111.025 62.325) (width 0.25) (layer "F.Cu") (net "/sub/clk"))
 (via (at 128.7319 62.3401) (size 0.9) (drill 0.45) (layers "F.Cu" "B.Cu") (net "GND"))
 (via (at 128.404595 61.168839) (size 0.8) (drill 0.48) (layers "F.Cu" "B.Cu") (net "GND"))
 (via (at 135.525302 62.953661) (size 0.8) (drill 0.48) (layers "F.Cu" "B.Cu") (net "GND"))
 (via (at 121.611193 60.555278) (size 0.9) (drill 0.45) (layers "F.Cu" "B.Cu") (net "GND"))
 (via (at 116.470518 59.199499) (size 0.8) (drill 0.48) (layers "F.Cu" "B.Cu") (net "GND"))
 (segment (start 117.966117 57.116117) (end 113.466117 57.116117) (width 0.35) (layer "B.Cu") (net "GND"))
 (segment (start 125.086824 58.900939) (end 120.586824 58.900939) (width 0.35) (layer "B.Cu") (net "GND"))
 (arc (start 118.85 56.75) (mid 118.444471 57.020966) (end 117.966117 57.116117) (width 0.35) (layer "B.Cu") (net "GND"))
 (arc (start 125.970707 58.534822) (mid 125.565178 58.805788) (end 125.086824 58.900939) (width 0.35) (layer "B.Cu") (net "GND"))
 (via (at 131.251828 55.811735) (size 0.9) (drill 0.54) (layers "F.Cu" "B.Cu") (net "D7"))
 (via (at 124.131121 54.026913) (size 0.9) (drill 0.54) (layers "F.Cu" "B.Cu") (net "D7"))
 (via (at 109.349811 57.414677) (size 0.8) (drill 0.48) (layers "F.Cu" "B.Cu") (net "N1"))
 (segment (start 119.180766 74.951086) (end 119.180766 72.451086) (width 0.35) (layer "B.Cu") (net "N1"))
 (segment (start 112.060059 70.666264) (end 112.060059 67.666264) (width 0.35) (layer "B.Cu") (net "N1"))
 (segment (start 119.180766 72.451086) (end 119.180766 69.451086) (width 0.35) (layer "B.Cu") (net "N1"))
 (segment (start 120.034319 69.097533) (end 121.534319 70.597533) (width 0.35) (layer "B.Cu") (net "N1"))
 (segment (start 112.913612 67.312711) (end 114.413612 68.812711) (width 0.35) (layer "B.Cu") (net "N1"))
 (segment (start 112.060059 73.166264) (end 112.060059 70.666264) (width 0.35) (layer "B.Cu") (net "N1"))
 (arc (start 110.120707 71.134822) (mid 110.916202 71.464327) (end 111.245707 72.259822) (width 0.15) (layer "B.Cu") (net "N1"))
 (arc (start 103 69.35) (mid 103.795495 69.679505) (end 104.125 70.475) (width 0.15) (layer "B.Cu") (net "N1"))
 (arc (start 112.060059 67.666264) (mid 112.368717 67.204324) (end 112.913612 67.312711) (width 0.35) (layer "B.Cu") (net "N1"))
 (arc (start 111.4 64.45) (mid 113.594214 65.916127) (end 113.079379 68.504379) (width 0.35) (layer "B.Cu") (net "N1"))
 (arc (start 104.125 70.475) (mid 103.502602 71.977602) (end 102 72.6) (width 0.15) (locked yes) (layer "B.Cu") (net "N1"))
 (arc (start 119.180766 69.451086) (mid 119.489424 68.989146) (end 120.034319 69.097533) (width 0.35) (layer "B.Cu") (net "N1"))
 (arc (start 118.520707 66.234822) (mid 120.714921 67.700949) (end 120.200086 70.289201) (width 0.35) (layer "B.Cu") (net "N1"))
 (segment (start 105.955293 61.168178) (end 104.455293 61.168178) (width 0.2) (layer "B.Cu") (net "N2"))
 (segment (start 115.576 62.953) (end 113.076 62.953) (width 0.2) (layer "B.Cu") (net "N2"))
 (segment (start 108.455293 61.168178) (end 105.955293 61.168178) (width 0.2) (layer "B.Cu") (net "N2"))
 (segment (start 113.076 62.953) (end 111.576 62.953) (width 0.2) (layer "B.Cu") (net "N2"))
 (arc (start 104.455293 61.168178) (mid 103.785597 61.034967) (end 103.217856 60.655615) (width 0.2) (layer "B.Cu") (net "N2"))
 (arc (start 111.576 62.953) (mid 110.906304 62.819789) (end 110.338563 62.440437) (width 0.2) (layer "B.Cu") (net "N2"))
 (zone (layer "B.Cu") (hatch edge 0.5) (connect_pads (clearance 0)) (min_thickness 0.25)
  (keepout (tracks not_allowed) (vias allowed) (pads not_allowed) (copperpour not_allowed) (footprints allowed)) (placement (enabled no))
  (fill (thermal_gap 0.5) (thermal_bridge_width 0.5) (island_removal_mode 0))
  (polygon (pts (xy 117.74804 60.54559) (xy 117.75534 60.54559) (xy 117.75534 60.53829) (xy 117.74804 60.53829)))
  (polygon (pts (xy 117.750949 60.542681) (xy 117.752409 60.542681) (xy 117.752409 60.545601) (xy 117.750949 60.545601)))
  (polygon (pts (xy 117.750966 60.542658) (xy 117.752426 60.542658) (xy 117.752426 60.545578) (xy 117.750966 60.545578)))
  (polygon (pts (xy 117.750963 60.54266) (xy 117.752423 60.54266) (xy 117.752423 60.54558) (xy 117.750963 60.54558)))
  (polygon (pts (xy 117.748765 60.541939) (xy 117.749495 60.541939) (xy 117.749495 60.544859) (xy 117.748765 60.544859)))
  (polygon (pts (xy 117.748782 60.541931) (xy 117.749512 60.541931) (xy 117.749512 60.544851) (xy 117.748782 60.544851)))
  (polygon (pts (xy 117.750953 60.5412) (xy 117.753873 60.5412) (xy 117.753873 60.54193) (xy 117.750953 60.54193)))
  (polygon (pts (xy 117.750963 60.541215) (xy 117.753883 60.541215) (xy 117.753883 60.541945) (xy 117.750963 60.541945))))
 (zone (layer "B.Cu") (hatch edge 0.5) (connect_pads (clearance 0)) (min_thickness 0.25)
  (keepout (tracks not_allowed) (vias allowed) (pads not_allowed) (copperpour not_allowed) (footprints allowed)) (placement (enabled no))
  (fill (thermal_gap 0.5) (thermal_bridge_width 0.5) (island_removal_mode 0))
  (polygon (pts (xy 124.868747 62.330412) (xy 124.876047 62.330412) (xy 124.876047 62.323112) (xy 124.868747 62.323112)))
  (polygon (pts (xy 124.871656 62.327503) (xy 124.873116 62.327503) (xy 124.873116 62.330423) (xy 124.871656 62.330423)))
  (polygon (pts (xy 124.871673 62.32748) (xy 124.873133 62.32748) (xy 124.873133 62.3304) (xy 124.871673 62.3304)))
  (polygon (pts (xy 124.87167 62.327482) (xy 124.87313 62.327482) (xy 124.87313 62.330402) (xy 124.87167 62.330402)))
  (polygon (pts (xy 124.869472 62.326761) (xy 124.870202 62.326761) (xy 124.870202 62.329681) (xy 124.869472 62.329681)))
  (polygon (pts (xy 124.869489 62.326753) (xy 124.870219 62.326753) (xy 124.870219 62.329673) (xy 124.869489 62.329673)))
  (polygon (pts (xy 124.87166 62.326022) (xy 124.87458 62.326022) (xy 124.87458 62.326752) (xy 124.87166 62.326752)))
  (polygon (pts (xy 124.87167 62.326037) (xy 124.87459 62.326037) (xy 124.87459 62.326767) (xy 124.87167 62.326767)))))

